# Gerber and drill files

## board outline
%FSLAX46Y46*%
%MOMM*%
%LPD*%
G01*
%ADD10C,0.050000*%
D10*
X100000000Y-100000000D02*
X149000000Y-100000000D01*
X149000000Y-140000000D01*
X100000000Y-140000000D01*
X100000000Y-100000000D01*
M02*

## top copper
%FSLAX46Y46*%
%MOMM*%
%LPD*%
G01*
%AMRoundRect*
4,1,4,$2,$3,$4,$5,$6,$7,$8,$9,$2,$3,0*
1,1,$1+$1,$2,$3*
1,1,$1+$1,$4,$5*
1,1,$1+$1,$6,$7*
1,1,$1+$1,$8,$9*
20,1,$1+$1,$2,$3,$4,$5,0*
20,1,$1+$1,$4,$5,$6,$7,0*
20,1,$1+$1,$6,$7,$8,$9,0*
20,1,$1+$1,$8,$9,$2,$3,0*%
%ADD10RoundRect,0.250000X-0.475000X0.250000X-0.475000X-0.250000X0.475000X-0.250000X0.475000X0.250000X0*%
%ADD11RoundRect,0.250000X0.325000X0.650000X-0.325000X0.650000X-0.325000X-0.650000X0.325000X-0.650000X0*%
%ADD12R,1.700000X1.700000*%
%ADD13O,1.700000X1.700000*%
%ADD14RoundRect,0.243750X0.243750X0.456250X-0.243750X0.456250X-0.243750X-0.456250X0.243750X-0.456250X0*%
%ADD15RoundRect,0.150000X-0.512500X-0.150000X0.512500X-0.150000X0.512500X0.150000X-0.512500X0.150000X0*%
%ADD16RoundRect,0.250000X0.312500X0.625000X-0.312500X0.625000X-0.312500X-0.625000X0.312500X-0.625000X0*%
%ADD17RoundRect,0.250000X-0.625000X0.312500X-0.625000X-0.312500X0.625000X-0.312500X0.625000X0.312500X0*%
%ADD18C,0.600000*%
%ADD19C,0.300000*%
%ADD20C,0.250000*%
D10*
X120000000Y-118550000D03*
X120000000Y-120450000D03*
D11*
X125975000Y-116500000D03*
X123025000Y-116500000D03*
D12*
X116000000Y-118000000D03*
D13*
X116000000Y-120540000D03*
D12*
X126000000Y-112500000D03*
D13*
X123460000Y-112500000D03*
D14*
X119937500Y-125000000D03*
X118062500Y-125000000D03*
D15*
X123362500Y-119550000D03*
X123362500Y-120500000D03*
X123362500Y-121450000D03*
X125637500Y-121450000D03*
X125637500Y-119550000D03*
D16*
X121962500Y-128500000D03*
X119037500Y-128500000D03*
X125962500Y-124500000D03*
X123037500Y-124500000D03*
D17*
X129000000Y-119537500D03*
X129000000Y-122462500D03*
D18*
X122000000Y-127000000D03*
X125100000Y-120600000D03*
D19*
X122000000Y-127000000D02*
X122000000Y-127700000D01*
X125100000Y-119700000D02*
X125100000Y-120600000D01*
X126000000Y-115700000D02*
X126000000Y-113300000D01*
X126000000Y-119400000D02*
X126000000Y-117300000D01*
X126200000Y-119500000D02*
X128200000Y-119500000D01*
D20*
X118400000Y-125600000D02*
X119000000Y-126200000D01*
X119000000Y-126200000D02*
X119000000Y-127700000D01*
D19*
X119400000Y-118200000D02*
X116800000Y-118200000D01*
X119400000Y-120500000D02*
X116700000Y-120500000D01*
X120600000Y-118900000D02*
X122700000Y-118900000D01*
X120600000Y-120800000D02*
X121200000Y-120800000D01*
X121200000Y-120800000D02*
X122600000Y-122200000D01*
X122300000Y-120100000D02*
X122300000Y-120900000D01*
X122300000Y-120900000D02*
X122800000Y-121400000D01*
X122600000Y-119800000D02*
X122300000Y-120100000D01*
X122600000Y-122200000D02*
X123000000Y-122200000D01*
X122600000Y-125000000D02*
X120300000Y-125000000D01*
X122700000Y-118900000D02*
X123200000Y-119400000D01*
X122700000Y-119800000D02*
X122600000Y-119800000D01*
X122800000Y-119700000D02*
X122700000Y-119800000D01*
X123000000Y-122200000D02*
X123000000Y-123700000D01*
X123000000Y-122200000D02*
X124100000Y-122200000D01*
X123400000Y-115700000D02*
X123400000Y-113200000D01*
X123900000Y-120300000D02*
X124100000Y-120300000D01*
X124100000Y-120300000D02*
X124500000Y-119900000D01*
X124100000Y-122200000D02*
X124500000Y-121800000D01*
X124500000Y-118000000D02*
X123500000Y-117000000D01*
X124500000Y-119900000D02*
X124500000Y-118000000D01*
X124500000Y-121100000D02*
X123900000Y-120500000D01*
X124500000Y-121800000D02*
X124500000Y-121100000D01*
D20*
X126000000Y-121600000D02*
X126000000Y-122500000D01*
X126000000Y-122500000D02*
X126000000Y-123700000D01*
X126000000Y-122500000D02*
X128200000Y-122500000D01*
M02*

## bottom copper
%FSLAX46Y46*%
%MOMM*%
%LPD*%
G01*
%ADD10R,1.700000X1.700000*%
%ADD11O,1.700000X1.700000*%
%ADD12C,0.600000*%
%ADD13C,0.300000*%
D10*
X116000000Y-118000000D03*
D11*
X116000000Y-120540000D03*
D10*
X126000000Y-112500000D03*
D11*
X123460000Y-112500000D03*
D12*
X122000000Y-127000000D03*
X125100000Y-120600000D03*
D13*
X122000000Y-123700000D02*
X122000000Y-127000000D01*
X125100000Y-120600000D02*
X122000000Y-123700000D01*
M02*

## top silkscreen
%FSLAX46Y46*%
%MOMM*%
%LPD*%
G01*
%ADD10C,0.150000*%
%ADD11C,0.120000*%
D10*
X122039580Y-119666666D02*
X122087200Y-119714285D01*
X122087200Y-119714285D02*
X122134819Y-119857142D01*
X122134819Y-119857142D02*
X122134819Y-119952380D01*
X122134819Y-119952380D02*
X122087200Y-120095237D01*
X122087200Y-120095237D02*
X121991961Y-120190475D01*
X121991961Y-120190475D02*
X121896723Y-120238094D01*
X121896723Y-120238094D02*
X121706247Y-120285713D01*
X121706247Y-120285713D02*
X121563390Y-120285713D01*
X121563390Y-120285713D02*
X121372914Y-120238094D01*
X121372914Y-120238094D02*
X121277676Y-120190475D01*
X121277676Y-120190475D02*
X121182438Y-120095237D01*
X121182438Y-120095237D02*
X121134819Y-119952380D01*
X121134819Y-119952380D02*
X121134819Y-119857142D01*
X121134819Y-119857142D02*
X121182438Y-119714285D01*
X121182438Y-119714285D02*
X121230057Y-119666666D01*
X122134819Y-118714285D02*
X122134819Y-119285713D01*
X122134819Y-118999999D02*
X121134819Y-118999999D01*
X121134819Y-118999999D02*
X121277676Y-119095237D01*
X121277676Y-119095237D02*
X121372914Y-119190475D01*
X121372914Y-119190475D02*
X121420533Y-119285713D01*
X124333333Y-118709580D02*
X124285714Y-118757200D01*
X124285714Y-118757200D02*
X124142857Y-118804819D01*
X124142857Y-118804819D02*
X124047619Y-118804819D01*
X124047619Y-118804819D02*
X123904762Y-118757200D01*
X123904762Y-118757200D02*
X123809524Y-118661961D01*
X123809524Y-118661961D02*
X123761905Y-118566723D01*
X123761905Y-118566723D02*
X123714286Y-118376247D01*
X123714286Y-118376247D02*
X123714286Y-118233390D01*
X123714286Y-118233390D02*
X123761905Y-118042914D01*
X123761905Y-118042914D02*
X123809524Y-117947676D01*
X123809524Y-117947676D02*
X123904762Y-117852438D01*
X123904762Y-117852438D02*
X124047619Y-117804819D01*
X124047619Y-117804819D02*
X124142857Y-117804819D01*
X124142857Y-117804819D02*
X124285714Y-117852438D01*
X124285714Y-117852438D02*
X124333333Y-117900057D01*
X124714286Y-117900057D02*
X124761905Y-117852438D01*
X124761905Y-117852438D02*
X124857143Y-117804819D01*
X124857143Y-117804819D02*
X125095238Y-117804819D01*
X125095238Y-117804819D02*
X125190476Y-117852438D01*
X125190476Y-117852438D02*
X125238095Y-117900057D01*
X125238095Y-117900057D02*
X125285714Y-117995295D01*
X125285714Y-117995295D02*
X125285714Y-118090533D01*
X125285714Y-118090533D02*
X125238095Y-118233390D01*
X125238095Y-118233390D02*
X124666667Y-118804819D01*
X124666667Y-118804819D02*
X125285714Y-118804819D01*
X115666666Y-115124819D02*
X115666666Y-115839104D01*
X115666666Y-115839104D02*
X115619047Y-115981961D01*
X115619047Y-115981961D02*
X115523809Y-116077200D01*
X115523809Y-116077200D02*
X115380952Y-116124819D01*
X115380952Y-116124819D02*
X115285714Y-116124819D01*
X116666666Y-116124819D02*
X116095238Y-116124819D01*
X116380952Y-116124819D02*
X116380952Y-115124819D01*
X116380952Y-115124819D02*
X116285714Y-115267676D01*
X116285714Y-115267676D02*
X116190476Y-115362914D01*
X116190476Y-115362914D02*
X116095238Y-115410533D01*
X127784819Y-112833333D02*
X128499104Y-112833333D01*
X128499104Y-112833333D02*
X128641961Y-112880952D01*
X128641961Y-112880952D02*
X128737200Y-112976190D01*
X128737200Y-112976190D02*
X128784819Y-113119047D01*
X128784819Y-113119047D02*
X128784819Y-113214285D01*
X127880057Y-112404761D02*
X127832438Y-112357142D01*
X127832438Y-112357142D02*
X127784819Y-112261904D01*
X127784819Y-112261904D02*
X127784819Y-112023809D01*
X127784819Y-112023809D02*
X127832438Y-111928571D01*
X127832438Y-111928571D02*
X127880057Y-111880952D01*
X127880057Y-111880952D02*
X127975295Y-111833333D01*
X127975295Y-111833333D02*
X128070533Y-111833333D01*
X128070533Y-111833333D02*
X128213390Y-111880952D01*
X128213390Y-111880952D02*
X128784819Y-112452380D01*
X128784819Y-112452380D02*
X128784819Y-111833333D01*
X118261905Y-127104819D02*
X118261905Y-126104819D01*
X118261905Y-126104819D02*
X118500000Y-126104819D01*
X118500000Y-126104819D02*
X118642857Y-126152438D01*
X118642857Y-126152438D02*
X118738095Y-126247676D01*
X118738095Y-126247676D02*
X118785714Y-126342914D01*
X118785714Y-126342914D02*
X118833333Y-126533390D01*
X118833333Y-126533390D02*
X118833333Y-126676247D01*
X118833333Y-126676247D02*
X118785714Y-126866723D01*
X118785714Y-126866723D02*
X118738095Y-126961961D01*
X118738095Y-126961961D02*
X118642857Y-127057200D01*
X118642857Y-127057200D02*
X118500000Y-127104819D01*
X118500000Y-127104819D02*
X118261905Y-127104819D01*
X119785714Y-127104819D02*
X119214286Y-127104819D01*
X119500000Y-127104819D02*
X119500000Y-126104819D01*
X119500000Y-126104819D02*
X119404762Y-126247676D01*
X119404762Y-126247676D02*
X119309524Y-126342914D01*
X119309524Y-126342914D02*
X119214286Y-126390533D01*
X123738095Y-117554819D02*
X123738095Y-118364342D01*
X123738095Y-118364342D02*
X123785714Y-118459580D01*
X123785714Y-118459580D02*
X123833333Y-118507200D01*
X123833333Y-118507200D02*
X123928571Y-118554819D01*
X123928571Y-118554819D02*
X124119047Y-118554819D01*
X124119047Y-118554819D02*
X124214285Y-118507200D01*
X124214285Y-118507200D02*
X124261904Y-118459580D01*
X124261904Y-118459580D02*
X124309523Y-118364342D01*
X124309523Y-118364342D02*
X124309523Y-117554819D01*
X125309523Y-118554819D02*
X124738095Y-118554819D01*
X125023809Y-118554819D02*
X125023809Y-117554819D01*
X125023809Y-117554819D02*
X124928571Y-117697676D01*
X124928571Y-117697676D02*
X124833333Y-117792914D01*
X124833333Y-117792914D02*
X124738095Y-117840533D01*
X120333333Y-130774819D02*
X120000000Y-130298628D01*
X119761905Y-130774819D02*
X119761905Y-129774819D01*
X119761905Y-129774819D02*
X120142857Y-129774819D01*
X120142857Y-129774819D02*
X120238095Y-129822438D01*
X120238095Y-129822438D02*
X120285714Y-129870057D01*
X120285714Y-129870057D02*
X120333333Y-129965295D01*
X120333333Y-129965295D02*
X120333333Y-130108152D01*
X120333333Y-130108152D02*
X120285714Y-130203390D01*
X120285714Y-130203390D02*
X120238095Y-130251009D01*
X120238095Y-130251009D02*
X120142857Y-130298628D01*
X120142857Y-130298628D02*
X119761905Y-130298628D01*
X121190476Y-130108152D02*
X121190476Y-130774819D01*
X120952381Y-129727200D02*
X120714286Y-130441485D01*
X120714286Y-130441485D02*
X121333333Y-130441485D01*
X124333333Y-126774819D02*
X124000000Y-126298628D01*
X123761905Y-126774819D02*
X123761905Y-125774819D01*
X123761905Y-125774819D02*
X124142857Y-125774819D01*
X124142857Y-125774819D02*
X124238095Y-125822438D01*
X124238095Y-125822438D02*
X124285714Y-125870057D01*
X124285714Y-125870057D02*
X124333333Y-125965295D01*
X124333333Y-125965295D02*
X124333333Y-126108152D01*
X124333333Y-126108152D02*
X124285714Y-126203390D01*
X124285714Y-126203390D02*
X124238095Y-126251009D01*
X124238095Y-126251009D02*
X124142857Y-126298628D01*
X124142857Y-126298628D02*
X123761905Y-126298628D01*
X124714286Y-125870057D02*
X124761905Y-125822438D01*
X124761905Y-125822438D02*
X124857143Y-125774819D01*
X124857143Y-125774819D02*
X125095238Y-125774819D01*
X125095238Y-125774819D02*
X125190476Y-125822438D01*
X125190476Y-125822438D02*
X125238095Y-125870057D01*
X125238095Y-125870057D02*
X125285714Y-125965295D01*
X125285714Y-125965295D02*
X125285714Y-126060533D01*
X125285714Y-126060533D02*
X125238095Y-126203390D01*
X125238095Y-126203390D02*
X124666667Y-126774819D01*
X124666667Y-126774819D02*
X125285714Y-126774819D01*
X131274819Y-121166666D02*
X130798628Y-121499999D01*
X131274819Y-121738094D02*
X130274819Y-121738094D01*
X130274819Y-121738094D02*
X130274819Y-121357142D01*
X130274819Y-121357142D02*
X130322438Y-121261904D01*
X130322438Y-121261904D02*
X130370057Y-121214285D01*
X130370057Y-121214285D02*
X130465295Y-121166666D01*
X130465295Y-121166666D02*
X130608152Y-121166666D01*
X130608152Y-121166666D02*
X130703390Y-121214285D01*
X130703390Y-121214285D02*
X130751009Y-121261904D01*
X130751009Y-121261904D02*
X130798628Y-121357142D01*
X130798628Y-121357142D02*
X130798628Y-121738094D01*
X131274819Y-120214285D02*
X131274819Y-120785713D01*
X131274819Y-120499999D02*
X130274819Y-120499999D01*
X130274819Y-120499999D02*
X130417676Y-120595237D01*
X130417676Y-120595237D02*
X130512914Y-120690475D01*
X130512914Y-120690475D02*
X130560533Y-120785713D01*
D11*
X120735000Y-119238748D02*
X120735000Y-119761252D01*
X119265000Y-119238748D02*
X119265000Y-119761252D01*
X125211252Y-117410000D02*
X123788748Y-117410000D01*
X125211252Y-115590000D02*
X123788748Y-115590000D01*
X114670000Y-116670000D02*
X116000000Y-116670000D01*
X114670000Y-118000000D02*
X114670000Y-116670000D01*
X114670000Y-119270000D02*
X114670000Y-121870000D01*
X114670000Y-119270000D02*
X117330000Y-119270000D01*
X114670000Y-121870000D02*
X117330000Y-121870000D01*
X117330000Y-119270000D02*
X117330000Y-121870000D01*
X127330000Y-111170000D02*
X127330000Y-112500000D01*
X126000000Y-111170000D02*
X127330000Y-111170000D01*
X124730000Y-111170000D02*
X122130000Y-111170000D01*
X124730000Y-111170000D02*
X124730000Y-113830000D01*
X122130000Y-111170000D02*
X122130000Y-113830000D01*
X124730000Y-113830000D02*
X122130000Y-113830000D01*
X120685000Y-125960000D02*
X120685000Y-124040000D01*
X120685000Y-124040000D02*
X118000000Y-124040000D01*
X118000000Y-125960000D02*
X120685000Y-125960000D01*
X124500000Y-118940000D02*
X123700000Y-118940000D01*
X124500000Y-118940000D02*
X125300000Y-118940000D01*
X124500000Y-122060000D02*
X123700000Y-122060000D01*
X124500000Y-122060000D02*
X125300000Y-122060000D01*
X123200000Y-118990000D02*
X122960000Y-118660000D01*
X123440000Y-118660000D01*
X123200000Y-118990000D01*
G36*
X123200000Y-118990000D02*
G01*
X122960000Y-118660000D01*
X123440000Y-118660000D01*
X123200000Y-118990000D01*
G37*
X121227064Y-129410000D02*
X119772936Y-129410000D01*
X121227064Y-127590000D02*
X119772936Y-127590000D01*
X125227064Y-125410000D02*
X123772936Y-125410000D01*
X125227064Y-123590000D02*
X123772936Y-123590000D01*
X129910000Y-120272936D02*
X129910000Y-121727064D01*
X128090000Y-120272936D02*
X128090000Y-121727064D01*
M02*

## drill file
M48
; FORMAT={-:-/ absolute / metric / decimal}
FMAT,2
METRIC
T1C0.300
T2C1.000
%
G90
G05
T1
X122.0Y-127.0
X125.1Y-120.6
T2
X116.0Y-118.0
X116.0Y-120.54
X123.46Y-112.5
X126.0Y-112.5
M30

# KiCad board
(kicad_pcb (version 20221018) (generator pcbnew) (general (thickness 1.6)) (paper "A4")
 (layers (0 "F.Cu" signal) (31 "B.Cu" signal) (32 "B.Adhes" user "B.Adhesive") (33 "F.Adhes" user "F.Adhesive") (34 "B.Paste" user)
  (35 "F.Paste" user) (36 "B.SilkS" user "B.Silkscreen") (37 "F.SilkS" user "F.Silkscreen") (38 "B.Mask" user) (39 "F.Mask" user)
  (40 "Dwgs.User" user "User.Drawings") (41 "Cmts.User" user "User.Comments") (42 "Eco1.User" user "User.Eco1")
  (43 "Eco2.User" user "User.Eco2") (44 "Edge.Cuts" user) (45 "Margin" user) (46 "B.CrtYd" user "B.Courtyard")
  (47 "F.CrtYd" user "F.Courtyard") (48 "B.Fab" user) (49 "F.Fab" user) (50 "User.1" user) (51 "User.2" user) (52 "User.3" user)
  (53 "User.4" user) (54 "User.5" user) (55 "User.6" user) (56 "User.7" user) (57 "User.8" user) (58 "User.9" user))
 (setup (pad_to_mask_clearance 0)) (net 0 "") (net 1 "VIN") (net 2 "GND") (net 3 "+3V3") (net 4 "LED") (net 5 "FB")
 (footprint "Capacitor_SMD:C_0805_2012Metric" (layer "F.Cu") (at 120 119.5 -90)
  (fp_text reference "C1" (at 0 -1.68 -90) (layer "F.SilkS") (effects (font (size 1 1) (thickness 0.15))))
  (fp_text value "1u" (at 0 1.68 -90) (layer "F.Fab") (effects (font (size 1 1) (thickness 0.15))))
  (fp_line (start -0.261252 -0.735) (end 0.261252 -0.735) (stroke (width 0.12) (type solid)) (layer "F.SilkS"))
  (fp_line (start -0.261252 0.735) (end 0.261252 0.735) (stroke (width 0.12) (type solid)) (layer "F.SilkS"))
  (pad "1" smd roundrect (at -0.95 0 270) (size 1 1.45) (layers "F.Cu" "F.Paste" "F.Mask") (roundrect_rratio 0.25) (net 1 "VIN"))
  (pad "2" smd roundrect (at 0.95 0 270) (size 1 1.45) (layers "F.Cu" "F.Paste" "F.Mask") (roundrect_rratio 0.25) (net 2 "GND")))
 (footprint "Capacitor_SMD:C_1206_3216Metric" (layer "F.Cu") (at 124.5 116.5 180)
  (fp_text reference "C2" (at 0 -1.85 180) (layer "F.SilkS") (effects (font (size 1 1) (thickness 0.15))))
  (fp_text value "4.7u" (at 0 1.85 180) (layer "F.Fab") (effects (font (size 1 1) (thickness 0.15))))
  (fp_line (start -0.711252 -0.91) (end 0.711252 -0.91) (stroke (width 0.12) (type solid)) (layer "F.SilkS"))
  (fp_line (start -0.711252 0.91) (end 0.711252 0.91) (stroke (width 0.12) (type solid)) (layer "F.SilkS"))
  (pad "1" smd roundrect (at -1.475 0 180) (size 1.15 1.8) (layers "F.Cu" "F.Paste" "F.Mask") (roundrect_rratio 0.217391) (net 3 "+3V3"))
  (pad "2" smd roundrect (at 1.475 0 180) (size 1.15 1.8) (layers "F.Cu" "F.Paste" "F.Mask") (roundrect_rratio 0.217391) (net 2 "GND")))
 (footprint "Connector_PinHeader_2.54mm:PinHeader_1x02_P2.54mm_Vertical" (layer "F.Cu") (at 116 118)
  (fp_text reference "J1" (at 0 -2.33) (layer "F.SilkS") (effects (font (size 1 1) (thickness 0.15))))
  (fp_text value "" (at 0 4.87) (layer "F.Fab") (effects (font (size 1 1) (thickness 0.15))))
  (fp_line (start -1.33 -1.33) (end 0 -1.33) (stroke (width 0.12) (type solid)) (layer "F.SilkS"))
  (fp_line (start -1.33 0) (end -1.33 -1.33) (stroke (width 0.12) (type solid)) (layer "F.SilkS"))
  (fp_line (start -1.33 1.27) (end -1.33 3.87) (stroke (width 0.12) (type solid)) (layer "F.SilkS"))
  (fp_line (start -1.33 1.27) (end 1.33 1.27) (stroke (width 0.12) (type solid)) (layer "F.SilkS"))
  (fp_line (start -1.33 3.87) (end 1.33 3.87) (stroke (width 0.12) (type solid)) (layer "F.SilkS"))
  (fp_line (start 1.33 1.27) (end 1.33 3.87) (stroke (width 0.12) (type solid)) (layer "F.SilkS"))
  (pad "1" thru_hole rect (at 0 0) (size 1.7 1.7) (drill 1) (layers "*.Cu" "*.Mask") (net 1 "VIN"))
  (pad "2" thru_hole oval (at 0 2.54) (size 1.7 1.7) (drill 1) (layers "*.Cu" "*.Mask") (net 2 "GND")))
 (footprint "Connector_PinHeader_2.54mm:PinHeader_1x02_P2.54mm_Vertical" (layer "F.Cu") (at 126 112.5 -90)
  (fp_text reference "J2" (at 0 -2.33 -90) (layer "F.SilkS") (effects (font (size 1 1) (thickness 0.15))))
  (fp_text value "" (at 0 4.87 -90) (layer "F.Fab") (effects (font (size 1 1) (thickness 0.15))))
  (fp_line (start -1.33 -1.33) (end 0 -1.33) (stroke (width 0.12) (type solid)) (layer "F.SilkS"))
  (fp_line (start -1.33 0) (end -1.33 -1.33) (stroke (width 0.12) (type solid)) (layer "F.SilkS"))
  (fp_line (start -1.33 1.27) (end -1.33 3.87) (stroke (width 0.12) (type solid)) (layer "F.SilkS"))
  (fp_line (start -1.33 1.27) (end 1.33 1.27) (stroke (width 0.12) (type solid)) (layer "F.SilkS"))
  (fp_line (start -1.33 3.87) (end 1.33 3.87) (stroke (width 0.12) (type solid)) (layer "F.SilkS"))
  (fp_line (start 1.33 1.27) (end 1.33 3.87) (stroke (width 0.12) (type solid)) (layer "F.SilkS"))
  (pad "1" thru_hole rect (at 0 0 270) (size 1.7 1.7) (drill 1) (layers "*.Cu" "*.Mask") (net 3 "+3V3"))
  (pad "2" thru_hole oval (at 0 2.54 270) (size 1.7 1.7) (drill 1) (layers "*.Cu" "*.Mask") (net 2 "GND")))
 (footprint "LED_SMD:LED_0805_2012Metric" (layer "F.Cu") (at 119 125 180)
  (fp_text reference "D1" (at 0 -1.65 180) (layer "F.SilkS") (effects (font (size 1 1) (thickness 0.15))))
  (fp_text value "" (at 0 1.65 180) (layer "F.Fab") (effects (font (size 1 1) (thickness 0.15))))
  (fp_line (start -1.685 -0.96) (end -1.685 0.96) (stroke (width 0.12) (type solid)) (layer "F.SilkS"))
  (fp_line (start -1.685 0.96) (end 1 0.96) (stroke (width 0.12) (type solid)) (layer "F.SilkS"))
  (fp_line (start 1 -0.96) (end -1.685 -0.96) (stroke (width 0.12) (type solid)) (layer "F.SilkS"))
  (pad "1" smd roundrect (at -0.9375 0 180) (size 0.975 1.4) (layers "F.Cu" "F.Paste" "F.Mask") (roundrect_rratio 0.25) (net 2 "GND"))
  (pad "2" smd roundrect (at 0.9375 0 180) (size 0.975 1.4) (layers "F.Cu" "F.Paste" "F.Mask") (roundrect_rratio 0.25) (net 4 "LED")))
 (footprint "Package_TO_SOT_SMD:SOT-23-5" (layer "F.Cu") (at 124.5 120.5)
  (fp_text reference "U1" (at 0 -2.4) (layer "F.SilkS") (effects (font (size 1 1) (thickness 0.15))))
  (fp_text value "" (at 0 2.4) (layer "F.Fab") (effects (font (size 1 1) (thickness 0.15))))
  (fp_line (start 0 -1.56) (end -0.8 -1.56) (stroke (width 0.12) (type solid)) (layer "F.SilkS"))
  (fp_line (start 0 -1.56) (end 0.8 -1.56) (stroke (width 0.12) (type solid)) (layer "F.SilkS"))
  (fp_line (start 0 1.56) (end -0.8 1.56) (stroke (width 0.12) (type solid)) (layer "F.SilkS"))
  (fp_line (start 0 1.56) (end 0.8 1.56) (stroke (width 0.12) (type solid)) (layer "F.SilkS"))
  (fp_poly
   (pts (xy -1.3 -1.51) (xy -1.54 -1.84) (xy -1.06 -1.84) (xy -1.3 -1.51)) (stroke (width 0.12) (type solid)) (fill solid) (layer "F.SilkS"))
  (pad "1" smd roundrect (at -1.1375 -0.95) (size 1.325 0.6) (layers "F.Cu" "F.Paste" "F.Mask") (roundrect_rratio 0.25) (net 1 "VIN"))
  (pad "2" smd roundrect (at -1.1375 0) (size 1.325 0.6) (layers "F.Cu" "F.Paste" "F.Mask") (roundrect_rratio 0.25) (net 2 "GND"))
  (pad "3" smd roundrect (at -1.1375 0.95) (size 1.325 0.6) (layers "F.Cu" "F.Paste" "F.Mask") (roundrect_rratio 0.25) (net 1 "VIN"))
  (pad "4" smd roundrect (at 1.1375 0.95) (size 1.325 0.6) (layers "F.Cu" "F.Paste" "F.Mask") (roundrect_rratio 0.25) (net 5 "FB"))
  (pad "5" smd roundrect (at 1.1375 -0.95) (size 1.325 0.6) (layers "F.Cu" "F.Paste" "F.Mask") (roundrect_rratio 0.25) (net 3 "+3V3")))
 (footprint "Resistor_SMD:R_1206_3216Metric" (layer "F.Cu") (at 120.5 128.5 180)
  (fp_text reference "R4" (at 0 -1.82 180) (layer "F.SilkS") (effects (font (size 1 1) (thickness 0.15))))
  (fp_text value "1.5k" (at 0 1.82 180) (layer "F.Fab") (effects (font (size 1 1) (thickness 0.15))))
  (fp_line (start -0.727064 -0.91) (end 0.727064 -0.91) (stroke (width 0.12) (type solid)) (layer "F.SilkS"))
  (fp_line (start -0.727064 0.91) (end 0.727064 0.91) (stroke (width 0.12) (type solid)) (layer "F.SilkS"))
  (pad "1" smd roundrect (at -1.4625 0 180) (size 1.125 1.75) (layers "F.Cu" "F.Paste" "F.Mask") (roundrect_rratio 0.222222) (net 3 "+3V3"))
  (pad "2" smd roundrect (at 1.4625 0 180) (size 1.125 1.75) (layers "F.Cu" "F.Paste" "F.Mask") (roundrect_rratio 0.222222) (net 4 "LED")))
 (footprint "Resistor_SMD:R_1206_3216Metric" (layer "F.Cu") (at 124.5 124.5 180)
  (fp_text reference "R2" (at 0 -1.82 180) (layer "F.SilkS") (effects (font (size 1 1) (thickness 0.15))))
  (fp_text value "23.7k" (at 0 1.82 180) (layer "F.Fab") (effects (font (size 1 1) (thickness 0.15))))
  (fp_line (start -0.727064 -0.91) (end 0.727064 -0.91) (stroke (width 0.12) (type solid)) (layer "F.SilkS"))
  (fp_line (start -0.727064 0.91) (end 0.727064 0.91) (stroke (width 0.12) (type solid)) (layer "F.SilkS"))
  (pad "1" smd roundrect (at -1.4625 0 180) (size 1.125 1.75) (layers "F.Cu" "F.Paste" "F.Mask") (roundrect_rratio 0.222222) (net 5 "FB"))
  (pad "2" smd roundrect (at 1.4625 0 180) (size 1.125 1.75) (layers "F.Cu" "F.Paste" "F.Mask") (roundrect_rratio 0.222222) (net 2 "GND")))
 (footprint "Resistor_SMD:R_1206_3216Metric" (layer "F.Cu") (at 129 121 -90)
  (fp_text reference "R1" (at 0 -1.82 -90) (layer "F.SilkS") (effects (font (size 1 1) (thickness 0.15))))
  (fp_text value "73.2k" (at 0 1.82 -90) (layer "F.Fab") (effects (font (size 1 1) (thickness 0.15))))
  (fp_line (start -0.727064 -0.91) (end 0.727064 -0.91) (stroke (width 0.12) (type solid)) (layer "F.SilkS"))
  (fp_line (start -0.727064 0.91) (end 0.727064 0.91) (stroke (width 0.12) (type solid)) (layer "F.SilkS"))
  (pad "1" smd roundrect (at -1.4625 0 270) (size 1.125 1.75) (layers "F.Cu" "F.Paste" "F.Mask") (roundrect_rratio 0.222222) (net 3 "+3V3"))
  (pad "2" smd roundrect (at 1.4625 0 270) (size 1.125 1.75) (layers "F.Cu" "F.Paste" "F.Mask") (roundrect_rratio 0.222222) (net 5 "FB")))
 (gr_rect (start 100 100) (end 149 140) (stroke (width 0.05) (type default)) (fill none) (layer "Edge.Cuts"))
 (segment (start 122 127) (end 122 127.7) (width 0.3) (layer "F.Cu") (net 3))
 (segment (start 125.1 119.7) (end 125.1 120.6) (width 0.3) (layer "F.Cu") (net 3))
 (segment (start 126 115.7) (end 126 113.3) (width 0.3) (layer "F.Cu") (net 3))
 (segment (start 126 119.4) (end 126 117.3) (width 0.3) (layer "F.Cu") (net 3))
 (segment (start 126.2 119.5) (end 128.2 119.5) (width 0.3) (layer "F.Cu") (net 3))
 (via (at 122 127) (size 0.6) (drill 0.3) (layers "F.Cu" "B.Cu") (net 3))
 (via (at 125.1 120.6) (size 0.6) (drill 0.3) (layers "F.Cu" "B.Cu") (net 3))
 (segment (start 118.4 125.6) (end 119 126.2) (width 0.25) (layer "F.Cu") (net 4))
 (segment (start 119 126.2) (end 119 127.7) (width 0.25) (layer "F.Cu") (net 4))
 (segment (start 119.4 118.2) (end 116.8 118.2) (width 0.3) (layer "F.Cu") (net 1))
 (segment (start 119.4 120.5) (end 116.7 120.5) (width 0.3) (layer "F.Cu") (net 2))
 (segment (start 120.6 118.9) (end 122.7 118.9) (width 0.3) (layer "F.Cu") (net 1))
 (segment (start 120.6 120.8) (end 121.2 120.8) (width 0.3) (layer "F.Cu") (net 2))
 (segment (start 121.2 120.8) (end 122.6 122.2) (width 0.3) (layer "F.Cu") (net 2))
 (segment (start 122 123.7) (end 122 127) (width 0.3) (layer "B.Cu") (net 3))
 (segment (start 122.3 120.1) (end 122.3 120.9) (width 0.3) (layer "F.Cu") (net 1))
 (segment (start 122.3 120.9) (end 122.8 121.4) (width 0.3) (layer "F.Cu") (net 1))
 (segment (start 122.6 119.8) (end 122.3 120.1) (width 0.3) (layer "F.Cu") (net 1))
 (segment (start 122.6 122.2) (end 123 122.2) (width 0.3) (layer "F.Cu") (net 2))
 (segment (start 122.6 125) (end 120.3 125) (width 0.3) (layer "F.Cu") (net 2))
 (segment (start 122.7 118.9) (end 123.2 119.4) (width 0.3) (layer "F.Cu") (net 1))
 (segment (start 122.7 119.8) (end 122.6 119.8) (width 0.3) (layer "F.Cu") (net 1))
 (segment (start 122.8 119.7) (end 122.7 119.8) (width 0.3) (layer "F.Cu") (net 1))
 (segment (start 123 122.2) (end 123 123.7) (width 0.3) (layer "F.Cu") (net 2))
 (segment (start 123 122.2) (end 124.1 122.2) (width 0.3) (layer "F.Cu") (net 2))
 (segment (start 123.4 115.7) (end 123.4 113.2) (width 0.3) (layer "F.Cu") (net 2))
 (segment (start 123.9 120.3) (end 124.1 120.3) (width 0.3) (layer "F.Cu") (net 2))
 (segment (start 124.1 120.3) (end 124.5 119.9) (width 0.3) (layer "F.Cu") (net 2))
 (segment (start 124.1 122.2) (end 124.5 121.8) (width 0.3) (layer "F.Cu") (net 2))
 (segment (start 124.5 118) (end 123.5 117) (width 0.3) (layer "F.Cu") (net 2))
 (segment (start 124.5 119.9) (end 124.5 118) (width 0.3) (layer "F.Cu") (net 2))
 (segment (start 124.5 121.1) (end 123.9 120.5) (width 0.3) (layer "F.Cu") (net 2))
 (segment (start 124.5 121.8) (end 124.5 121.1) (width 0.3) (layer "F.Cu") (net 2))
 (segment (start 125.1 120.6) (end 122 123.7) (width 0.3) (layer "B.Cu") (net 3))
 (segment (start 126 121.6) (end 126 122.5) (width 0.25) (layer "F.Cu") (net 5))
 (segment (start 126 122.5) (end 126 123.7) (width 0.25) (layer "F.Cu") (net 5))
 (segment (start 126 122.5) (end 128.2 122.5) (width 0.25) (layer "F.Cu") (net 5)))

